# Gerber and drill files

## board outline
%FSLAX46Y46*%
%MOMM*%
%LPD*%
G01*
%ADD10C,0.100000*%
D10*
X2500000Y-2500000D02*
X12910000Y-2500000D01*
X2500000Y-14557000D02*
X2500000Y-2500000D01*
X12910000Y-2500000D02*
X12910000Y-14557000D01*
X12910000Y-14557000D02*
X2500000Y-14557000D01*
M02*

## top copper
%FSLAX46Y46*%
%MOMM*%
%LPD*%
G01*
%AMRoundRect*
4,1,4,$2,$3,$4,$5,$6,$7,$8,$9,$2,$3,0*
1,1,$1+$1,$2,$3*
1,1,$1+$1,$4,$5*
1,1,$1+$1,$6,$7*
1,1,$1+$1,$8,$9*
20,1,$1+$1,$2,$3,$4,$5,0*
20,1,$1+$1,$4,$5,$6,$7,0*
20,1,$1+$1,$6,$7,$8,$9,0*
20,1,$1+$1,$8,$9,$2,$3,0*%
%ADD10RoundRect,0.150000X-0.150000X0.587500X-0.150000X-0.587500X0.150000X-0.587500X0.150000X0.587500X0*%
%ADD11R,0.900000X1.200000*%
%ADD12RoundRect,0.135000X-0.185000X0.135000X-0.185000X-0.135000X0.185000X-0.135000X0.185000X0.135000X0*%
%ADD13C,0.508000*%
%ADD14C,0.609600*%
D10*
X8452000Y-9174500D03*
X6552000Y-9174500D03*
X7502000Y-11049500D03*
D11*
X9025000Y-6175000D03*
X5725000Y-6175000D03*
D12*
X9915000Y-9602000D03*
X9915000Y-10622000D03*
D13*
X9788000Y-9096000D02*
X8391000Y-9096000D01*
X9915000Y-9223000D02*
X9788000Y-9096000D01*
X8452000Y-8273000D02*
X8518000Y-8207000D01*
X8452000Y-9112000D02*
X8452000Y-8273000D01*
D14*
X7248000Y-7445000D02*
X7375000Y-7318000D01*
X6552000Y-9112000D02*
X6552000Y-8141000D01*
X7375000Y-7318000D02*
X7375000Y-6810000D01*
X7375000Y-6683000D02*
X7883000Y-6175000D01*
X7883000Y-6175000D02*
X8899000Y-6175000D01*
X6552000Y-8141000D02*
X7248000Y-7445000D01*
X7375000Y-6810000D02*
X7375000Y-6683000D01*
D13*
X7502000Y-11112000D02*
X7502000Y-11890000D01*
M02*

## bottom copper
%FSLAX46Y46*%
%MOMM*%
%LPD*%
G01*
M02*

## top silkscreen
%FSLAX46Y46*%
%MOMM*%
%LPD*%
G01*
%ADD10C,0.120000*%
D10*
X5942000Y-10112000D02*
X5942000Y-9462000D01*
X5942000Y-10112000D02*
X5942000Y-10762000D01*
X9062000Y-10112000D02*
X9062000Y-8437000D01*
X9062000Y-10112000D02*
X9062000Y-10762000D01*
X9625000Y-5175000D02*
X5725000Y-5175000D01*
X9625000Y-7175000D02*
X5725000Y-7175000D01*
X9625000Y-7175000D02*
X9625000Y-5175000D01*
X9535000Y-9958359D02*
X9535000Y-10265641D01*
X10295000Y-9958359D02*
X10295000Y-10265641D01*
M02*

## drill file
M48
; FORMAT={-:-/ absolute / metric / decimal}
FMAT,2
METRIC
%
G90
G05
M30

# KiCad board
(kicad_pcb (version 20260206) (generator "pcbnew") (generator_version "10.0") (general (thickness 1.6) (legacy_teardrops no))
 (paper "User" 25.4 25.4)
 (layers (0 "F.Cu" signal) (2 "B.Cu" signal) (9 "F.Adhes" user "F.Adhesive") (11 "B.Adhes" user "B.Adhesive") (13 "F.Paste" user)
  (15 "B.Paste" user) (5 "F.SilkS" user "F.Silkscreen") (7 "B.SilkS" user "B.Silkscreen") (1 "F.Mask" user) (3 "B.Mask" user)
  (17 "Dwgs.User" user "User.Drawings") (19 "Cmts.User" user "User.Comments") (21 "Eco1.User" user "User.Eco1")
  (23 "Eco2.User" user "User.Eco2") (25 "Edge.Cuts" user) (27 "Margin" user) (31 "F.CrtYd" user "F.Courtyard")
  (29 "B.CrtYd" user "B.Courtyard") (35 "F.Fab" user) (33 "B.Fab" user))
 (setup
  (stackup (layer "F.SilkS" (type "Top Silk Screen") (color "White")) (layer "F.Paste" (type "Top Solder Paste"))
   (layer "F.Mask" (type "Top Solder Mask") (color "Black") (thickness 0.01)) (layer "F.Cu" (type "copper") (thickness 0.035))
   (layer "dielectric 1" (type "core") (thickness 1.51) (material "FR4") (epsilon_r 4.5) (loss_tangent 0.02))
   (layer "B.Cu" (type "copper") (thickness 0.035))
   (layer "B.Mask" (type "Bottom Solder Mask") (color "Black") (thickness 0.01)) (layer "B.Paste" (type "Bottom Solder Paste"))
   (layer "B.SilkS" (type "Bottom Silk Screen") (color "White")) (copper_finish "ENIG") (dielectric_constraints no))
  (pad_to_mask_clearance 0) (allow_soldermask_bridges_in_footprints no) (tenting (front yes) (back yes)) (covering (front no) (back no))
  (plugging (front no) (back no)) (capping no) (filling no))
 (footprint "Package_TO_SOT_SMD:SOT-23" (layer "F.Cu") (at 7.502 10.112 -90)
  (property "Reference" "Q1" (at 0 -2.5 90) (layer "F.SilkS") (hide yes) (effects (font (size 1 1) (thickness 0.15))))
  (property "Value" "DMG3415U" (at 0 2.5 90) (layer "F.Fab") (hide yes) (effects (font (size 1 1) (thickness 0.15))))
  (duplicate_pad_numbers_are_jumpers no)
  (fp_line (start 0 1.56) (end -0.65 1.56) (stroke (width 0.12) (type solid)) (layer "F.SilkS"))
  (fp_line (start 0 1.56) (end 0.65 1.56) (stroke (width 0.12) (type solid)) (layer "F.SilkS"))
  (fp_line (start 0 -1.56) (end -1.675 -1.56) (stroke (width 0.12) (type solid)) (layer "F.SilkS"))
  (fp_line (start 0 -1.56) (end 0.65 -1.56) (stroke (width 0.12) (type solid)) (layer "F.SilkS"))
  (pad "1" smd roundrect (at -0.9375 -0.95 270) (size 1.475 0.6) (layers "F.Cu" "F.Mask" "F.Paste") (roundrect_rratio 0.25) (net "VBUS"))
  (pad "2" smd roundrect (at -0.9375 0.95 270) (size 1.475 0.6) (layers "F.Cu" "F.Mask" "F.Paste") (roundrect_rratio 0.25) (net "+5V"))
  (pad "3" smd roundrect (at 0.9375 0 270) (size 1.475 0.6) (layers "F.Cu" "F.Mask" "F.Paste") (roundrect_rratio 0.25) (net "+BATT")))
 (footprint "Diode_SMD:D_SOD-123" (layer "F.Cu") (at 7.375 6.175 180)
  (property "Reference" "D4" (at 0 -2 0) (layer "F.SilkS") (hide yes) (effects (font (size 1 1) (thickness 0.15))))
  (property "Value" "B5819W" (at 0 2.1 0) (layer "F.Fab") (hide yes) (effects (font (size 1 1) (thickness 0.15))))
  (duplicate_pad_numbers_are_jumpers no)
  (fp_line (start -2.25 1) (end 1.65 1) (stroke (width 0.12) (type solid)) (layer "F.SilkS"))
  (fp_line (start -2.25 -1) (end 1.65 -1) (stroke (width 0.12) (type solid)) (layer "F.SilkS"))
  (fp_line (start -2.25 -1) (end -2.25 1) (stroke (width 0.12) (type solid)) (layer "F.SilkS"))
  (pad "1" smd rect (at -1.65 0 180) (size 0.9 1.2) (layers "F.Cu" "F.Mask" "F.Paste") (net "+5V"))
  (pad "2" smd rect (at 1.65 0 180) (size 0.9 1.2) (layers "F.Cu" "F.Mask" "F.Paste") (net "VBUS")))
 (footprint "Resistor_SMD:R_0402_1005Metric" (layer "F.Cu") (at 9.915 10.112 -90)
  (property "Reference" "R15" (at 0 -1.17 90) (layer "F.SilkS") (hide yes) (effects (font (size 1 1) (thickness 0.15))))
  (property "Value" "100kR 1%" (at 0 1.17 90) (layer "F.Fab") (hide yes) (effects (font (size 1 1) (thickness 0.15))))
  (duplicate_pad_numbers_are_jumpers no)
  (fp_line (start -0.153641 0.38) (end 0.153641 0.38) (stroke (width 0.12) (type solid)) (layer "F.SilkS"))
  (fp_line (start -0.153641 -0.38) (end 0.153641 -0.38) (stroke (width 0.12) (type solid)) (layer "F.SilkS"))
  (pad "1" smd roundrect (at -0.51 0 270) (size 0.54 0.64) (layers "F.Cu" "F.Mask" "F.Paste") (roundrect_rratio 0.25) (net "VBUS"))
  (pad "2" smd roundrect (at 0.51 0 270) (size 0.54 0.64) (layers "F.Cu" "F.Mask" "F.Paste") (roundrect_rratio 0.25) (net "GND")))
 (gr_line (start 2.5 2.5) (end 12.91 2.5) (stroke (width 0.1) (type default)) (layer "Edge.Cuts"))
 (gr_line (start 2.5 14.557) (end 2.5 2.5) (stroke (width 0.1) (type default)) (layer "Edge.Cuts"))
 (gr_line (start 12.91 2.5) (end 12.91 14.557) (stroke (width 0.1) (type default)) (layer "Edge.Cuts"))
 (gr_line (start 12.91 14.557) (end 2.5 14.557) (stroke (width 0.1) (type default)) (layer "Edge.Cuts"))
 (segment (start 9.788 9.096) (end 8.391 9.096) (width 0.508) (layer "F.Cu") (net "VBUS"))
 (segment (start 9.915 9.223) (end 9.788 9.096) (width 0.508) (layer "F.Cu") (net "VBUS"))
 (segment (start 8.452 8.273) (end 8.518 8.207) (width 0.508) (layer "F.Cu") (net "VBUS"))
 (segment (start 8.452 9.112) (end 8.452 8.273) (width 0.508) (layer "F.Cu") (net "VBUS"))
 (segment (start 7.248 7.445) (end 7.375 7.318) (width 0.6096) (layer "F.Cu") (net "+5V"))
 (segment (start 6.552 9.112) (end 6.552 8.141) (width 0.6096) (layer "F.Cu") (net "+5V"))
 (segment (start 7.375 7.318) (end 7.375 6.81) (width 0.6096) (layer "F.Cu") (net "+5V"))
 (segment (start 7.375 6.683) (end 7.883 6.175) (width 0.6096) (layer "F.Cu") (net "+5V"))
 (segment (start 7.883 6.175) (end 8.899 6.175) (width 0.6096) (layer "F.Cu") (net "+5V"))
 (segment (start 6.552 8.141) (end 7.248 7.445) (width 0.6096) (layer "F.Cu") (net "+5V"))
 (segment (start 7.375 6.81) (end 7.375 6.683) (width 0.6096) (layer "F.Cu") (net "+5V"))
 (segment (start 7.502 11.112) (end 7.502 11.89) (width 0.508) (layer "F.Cu") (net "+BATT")))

